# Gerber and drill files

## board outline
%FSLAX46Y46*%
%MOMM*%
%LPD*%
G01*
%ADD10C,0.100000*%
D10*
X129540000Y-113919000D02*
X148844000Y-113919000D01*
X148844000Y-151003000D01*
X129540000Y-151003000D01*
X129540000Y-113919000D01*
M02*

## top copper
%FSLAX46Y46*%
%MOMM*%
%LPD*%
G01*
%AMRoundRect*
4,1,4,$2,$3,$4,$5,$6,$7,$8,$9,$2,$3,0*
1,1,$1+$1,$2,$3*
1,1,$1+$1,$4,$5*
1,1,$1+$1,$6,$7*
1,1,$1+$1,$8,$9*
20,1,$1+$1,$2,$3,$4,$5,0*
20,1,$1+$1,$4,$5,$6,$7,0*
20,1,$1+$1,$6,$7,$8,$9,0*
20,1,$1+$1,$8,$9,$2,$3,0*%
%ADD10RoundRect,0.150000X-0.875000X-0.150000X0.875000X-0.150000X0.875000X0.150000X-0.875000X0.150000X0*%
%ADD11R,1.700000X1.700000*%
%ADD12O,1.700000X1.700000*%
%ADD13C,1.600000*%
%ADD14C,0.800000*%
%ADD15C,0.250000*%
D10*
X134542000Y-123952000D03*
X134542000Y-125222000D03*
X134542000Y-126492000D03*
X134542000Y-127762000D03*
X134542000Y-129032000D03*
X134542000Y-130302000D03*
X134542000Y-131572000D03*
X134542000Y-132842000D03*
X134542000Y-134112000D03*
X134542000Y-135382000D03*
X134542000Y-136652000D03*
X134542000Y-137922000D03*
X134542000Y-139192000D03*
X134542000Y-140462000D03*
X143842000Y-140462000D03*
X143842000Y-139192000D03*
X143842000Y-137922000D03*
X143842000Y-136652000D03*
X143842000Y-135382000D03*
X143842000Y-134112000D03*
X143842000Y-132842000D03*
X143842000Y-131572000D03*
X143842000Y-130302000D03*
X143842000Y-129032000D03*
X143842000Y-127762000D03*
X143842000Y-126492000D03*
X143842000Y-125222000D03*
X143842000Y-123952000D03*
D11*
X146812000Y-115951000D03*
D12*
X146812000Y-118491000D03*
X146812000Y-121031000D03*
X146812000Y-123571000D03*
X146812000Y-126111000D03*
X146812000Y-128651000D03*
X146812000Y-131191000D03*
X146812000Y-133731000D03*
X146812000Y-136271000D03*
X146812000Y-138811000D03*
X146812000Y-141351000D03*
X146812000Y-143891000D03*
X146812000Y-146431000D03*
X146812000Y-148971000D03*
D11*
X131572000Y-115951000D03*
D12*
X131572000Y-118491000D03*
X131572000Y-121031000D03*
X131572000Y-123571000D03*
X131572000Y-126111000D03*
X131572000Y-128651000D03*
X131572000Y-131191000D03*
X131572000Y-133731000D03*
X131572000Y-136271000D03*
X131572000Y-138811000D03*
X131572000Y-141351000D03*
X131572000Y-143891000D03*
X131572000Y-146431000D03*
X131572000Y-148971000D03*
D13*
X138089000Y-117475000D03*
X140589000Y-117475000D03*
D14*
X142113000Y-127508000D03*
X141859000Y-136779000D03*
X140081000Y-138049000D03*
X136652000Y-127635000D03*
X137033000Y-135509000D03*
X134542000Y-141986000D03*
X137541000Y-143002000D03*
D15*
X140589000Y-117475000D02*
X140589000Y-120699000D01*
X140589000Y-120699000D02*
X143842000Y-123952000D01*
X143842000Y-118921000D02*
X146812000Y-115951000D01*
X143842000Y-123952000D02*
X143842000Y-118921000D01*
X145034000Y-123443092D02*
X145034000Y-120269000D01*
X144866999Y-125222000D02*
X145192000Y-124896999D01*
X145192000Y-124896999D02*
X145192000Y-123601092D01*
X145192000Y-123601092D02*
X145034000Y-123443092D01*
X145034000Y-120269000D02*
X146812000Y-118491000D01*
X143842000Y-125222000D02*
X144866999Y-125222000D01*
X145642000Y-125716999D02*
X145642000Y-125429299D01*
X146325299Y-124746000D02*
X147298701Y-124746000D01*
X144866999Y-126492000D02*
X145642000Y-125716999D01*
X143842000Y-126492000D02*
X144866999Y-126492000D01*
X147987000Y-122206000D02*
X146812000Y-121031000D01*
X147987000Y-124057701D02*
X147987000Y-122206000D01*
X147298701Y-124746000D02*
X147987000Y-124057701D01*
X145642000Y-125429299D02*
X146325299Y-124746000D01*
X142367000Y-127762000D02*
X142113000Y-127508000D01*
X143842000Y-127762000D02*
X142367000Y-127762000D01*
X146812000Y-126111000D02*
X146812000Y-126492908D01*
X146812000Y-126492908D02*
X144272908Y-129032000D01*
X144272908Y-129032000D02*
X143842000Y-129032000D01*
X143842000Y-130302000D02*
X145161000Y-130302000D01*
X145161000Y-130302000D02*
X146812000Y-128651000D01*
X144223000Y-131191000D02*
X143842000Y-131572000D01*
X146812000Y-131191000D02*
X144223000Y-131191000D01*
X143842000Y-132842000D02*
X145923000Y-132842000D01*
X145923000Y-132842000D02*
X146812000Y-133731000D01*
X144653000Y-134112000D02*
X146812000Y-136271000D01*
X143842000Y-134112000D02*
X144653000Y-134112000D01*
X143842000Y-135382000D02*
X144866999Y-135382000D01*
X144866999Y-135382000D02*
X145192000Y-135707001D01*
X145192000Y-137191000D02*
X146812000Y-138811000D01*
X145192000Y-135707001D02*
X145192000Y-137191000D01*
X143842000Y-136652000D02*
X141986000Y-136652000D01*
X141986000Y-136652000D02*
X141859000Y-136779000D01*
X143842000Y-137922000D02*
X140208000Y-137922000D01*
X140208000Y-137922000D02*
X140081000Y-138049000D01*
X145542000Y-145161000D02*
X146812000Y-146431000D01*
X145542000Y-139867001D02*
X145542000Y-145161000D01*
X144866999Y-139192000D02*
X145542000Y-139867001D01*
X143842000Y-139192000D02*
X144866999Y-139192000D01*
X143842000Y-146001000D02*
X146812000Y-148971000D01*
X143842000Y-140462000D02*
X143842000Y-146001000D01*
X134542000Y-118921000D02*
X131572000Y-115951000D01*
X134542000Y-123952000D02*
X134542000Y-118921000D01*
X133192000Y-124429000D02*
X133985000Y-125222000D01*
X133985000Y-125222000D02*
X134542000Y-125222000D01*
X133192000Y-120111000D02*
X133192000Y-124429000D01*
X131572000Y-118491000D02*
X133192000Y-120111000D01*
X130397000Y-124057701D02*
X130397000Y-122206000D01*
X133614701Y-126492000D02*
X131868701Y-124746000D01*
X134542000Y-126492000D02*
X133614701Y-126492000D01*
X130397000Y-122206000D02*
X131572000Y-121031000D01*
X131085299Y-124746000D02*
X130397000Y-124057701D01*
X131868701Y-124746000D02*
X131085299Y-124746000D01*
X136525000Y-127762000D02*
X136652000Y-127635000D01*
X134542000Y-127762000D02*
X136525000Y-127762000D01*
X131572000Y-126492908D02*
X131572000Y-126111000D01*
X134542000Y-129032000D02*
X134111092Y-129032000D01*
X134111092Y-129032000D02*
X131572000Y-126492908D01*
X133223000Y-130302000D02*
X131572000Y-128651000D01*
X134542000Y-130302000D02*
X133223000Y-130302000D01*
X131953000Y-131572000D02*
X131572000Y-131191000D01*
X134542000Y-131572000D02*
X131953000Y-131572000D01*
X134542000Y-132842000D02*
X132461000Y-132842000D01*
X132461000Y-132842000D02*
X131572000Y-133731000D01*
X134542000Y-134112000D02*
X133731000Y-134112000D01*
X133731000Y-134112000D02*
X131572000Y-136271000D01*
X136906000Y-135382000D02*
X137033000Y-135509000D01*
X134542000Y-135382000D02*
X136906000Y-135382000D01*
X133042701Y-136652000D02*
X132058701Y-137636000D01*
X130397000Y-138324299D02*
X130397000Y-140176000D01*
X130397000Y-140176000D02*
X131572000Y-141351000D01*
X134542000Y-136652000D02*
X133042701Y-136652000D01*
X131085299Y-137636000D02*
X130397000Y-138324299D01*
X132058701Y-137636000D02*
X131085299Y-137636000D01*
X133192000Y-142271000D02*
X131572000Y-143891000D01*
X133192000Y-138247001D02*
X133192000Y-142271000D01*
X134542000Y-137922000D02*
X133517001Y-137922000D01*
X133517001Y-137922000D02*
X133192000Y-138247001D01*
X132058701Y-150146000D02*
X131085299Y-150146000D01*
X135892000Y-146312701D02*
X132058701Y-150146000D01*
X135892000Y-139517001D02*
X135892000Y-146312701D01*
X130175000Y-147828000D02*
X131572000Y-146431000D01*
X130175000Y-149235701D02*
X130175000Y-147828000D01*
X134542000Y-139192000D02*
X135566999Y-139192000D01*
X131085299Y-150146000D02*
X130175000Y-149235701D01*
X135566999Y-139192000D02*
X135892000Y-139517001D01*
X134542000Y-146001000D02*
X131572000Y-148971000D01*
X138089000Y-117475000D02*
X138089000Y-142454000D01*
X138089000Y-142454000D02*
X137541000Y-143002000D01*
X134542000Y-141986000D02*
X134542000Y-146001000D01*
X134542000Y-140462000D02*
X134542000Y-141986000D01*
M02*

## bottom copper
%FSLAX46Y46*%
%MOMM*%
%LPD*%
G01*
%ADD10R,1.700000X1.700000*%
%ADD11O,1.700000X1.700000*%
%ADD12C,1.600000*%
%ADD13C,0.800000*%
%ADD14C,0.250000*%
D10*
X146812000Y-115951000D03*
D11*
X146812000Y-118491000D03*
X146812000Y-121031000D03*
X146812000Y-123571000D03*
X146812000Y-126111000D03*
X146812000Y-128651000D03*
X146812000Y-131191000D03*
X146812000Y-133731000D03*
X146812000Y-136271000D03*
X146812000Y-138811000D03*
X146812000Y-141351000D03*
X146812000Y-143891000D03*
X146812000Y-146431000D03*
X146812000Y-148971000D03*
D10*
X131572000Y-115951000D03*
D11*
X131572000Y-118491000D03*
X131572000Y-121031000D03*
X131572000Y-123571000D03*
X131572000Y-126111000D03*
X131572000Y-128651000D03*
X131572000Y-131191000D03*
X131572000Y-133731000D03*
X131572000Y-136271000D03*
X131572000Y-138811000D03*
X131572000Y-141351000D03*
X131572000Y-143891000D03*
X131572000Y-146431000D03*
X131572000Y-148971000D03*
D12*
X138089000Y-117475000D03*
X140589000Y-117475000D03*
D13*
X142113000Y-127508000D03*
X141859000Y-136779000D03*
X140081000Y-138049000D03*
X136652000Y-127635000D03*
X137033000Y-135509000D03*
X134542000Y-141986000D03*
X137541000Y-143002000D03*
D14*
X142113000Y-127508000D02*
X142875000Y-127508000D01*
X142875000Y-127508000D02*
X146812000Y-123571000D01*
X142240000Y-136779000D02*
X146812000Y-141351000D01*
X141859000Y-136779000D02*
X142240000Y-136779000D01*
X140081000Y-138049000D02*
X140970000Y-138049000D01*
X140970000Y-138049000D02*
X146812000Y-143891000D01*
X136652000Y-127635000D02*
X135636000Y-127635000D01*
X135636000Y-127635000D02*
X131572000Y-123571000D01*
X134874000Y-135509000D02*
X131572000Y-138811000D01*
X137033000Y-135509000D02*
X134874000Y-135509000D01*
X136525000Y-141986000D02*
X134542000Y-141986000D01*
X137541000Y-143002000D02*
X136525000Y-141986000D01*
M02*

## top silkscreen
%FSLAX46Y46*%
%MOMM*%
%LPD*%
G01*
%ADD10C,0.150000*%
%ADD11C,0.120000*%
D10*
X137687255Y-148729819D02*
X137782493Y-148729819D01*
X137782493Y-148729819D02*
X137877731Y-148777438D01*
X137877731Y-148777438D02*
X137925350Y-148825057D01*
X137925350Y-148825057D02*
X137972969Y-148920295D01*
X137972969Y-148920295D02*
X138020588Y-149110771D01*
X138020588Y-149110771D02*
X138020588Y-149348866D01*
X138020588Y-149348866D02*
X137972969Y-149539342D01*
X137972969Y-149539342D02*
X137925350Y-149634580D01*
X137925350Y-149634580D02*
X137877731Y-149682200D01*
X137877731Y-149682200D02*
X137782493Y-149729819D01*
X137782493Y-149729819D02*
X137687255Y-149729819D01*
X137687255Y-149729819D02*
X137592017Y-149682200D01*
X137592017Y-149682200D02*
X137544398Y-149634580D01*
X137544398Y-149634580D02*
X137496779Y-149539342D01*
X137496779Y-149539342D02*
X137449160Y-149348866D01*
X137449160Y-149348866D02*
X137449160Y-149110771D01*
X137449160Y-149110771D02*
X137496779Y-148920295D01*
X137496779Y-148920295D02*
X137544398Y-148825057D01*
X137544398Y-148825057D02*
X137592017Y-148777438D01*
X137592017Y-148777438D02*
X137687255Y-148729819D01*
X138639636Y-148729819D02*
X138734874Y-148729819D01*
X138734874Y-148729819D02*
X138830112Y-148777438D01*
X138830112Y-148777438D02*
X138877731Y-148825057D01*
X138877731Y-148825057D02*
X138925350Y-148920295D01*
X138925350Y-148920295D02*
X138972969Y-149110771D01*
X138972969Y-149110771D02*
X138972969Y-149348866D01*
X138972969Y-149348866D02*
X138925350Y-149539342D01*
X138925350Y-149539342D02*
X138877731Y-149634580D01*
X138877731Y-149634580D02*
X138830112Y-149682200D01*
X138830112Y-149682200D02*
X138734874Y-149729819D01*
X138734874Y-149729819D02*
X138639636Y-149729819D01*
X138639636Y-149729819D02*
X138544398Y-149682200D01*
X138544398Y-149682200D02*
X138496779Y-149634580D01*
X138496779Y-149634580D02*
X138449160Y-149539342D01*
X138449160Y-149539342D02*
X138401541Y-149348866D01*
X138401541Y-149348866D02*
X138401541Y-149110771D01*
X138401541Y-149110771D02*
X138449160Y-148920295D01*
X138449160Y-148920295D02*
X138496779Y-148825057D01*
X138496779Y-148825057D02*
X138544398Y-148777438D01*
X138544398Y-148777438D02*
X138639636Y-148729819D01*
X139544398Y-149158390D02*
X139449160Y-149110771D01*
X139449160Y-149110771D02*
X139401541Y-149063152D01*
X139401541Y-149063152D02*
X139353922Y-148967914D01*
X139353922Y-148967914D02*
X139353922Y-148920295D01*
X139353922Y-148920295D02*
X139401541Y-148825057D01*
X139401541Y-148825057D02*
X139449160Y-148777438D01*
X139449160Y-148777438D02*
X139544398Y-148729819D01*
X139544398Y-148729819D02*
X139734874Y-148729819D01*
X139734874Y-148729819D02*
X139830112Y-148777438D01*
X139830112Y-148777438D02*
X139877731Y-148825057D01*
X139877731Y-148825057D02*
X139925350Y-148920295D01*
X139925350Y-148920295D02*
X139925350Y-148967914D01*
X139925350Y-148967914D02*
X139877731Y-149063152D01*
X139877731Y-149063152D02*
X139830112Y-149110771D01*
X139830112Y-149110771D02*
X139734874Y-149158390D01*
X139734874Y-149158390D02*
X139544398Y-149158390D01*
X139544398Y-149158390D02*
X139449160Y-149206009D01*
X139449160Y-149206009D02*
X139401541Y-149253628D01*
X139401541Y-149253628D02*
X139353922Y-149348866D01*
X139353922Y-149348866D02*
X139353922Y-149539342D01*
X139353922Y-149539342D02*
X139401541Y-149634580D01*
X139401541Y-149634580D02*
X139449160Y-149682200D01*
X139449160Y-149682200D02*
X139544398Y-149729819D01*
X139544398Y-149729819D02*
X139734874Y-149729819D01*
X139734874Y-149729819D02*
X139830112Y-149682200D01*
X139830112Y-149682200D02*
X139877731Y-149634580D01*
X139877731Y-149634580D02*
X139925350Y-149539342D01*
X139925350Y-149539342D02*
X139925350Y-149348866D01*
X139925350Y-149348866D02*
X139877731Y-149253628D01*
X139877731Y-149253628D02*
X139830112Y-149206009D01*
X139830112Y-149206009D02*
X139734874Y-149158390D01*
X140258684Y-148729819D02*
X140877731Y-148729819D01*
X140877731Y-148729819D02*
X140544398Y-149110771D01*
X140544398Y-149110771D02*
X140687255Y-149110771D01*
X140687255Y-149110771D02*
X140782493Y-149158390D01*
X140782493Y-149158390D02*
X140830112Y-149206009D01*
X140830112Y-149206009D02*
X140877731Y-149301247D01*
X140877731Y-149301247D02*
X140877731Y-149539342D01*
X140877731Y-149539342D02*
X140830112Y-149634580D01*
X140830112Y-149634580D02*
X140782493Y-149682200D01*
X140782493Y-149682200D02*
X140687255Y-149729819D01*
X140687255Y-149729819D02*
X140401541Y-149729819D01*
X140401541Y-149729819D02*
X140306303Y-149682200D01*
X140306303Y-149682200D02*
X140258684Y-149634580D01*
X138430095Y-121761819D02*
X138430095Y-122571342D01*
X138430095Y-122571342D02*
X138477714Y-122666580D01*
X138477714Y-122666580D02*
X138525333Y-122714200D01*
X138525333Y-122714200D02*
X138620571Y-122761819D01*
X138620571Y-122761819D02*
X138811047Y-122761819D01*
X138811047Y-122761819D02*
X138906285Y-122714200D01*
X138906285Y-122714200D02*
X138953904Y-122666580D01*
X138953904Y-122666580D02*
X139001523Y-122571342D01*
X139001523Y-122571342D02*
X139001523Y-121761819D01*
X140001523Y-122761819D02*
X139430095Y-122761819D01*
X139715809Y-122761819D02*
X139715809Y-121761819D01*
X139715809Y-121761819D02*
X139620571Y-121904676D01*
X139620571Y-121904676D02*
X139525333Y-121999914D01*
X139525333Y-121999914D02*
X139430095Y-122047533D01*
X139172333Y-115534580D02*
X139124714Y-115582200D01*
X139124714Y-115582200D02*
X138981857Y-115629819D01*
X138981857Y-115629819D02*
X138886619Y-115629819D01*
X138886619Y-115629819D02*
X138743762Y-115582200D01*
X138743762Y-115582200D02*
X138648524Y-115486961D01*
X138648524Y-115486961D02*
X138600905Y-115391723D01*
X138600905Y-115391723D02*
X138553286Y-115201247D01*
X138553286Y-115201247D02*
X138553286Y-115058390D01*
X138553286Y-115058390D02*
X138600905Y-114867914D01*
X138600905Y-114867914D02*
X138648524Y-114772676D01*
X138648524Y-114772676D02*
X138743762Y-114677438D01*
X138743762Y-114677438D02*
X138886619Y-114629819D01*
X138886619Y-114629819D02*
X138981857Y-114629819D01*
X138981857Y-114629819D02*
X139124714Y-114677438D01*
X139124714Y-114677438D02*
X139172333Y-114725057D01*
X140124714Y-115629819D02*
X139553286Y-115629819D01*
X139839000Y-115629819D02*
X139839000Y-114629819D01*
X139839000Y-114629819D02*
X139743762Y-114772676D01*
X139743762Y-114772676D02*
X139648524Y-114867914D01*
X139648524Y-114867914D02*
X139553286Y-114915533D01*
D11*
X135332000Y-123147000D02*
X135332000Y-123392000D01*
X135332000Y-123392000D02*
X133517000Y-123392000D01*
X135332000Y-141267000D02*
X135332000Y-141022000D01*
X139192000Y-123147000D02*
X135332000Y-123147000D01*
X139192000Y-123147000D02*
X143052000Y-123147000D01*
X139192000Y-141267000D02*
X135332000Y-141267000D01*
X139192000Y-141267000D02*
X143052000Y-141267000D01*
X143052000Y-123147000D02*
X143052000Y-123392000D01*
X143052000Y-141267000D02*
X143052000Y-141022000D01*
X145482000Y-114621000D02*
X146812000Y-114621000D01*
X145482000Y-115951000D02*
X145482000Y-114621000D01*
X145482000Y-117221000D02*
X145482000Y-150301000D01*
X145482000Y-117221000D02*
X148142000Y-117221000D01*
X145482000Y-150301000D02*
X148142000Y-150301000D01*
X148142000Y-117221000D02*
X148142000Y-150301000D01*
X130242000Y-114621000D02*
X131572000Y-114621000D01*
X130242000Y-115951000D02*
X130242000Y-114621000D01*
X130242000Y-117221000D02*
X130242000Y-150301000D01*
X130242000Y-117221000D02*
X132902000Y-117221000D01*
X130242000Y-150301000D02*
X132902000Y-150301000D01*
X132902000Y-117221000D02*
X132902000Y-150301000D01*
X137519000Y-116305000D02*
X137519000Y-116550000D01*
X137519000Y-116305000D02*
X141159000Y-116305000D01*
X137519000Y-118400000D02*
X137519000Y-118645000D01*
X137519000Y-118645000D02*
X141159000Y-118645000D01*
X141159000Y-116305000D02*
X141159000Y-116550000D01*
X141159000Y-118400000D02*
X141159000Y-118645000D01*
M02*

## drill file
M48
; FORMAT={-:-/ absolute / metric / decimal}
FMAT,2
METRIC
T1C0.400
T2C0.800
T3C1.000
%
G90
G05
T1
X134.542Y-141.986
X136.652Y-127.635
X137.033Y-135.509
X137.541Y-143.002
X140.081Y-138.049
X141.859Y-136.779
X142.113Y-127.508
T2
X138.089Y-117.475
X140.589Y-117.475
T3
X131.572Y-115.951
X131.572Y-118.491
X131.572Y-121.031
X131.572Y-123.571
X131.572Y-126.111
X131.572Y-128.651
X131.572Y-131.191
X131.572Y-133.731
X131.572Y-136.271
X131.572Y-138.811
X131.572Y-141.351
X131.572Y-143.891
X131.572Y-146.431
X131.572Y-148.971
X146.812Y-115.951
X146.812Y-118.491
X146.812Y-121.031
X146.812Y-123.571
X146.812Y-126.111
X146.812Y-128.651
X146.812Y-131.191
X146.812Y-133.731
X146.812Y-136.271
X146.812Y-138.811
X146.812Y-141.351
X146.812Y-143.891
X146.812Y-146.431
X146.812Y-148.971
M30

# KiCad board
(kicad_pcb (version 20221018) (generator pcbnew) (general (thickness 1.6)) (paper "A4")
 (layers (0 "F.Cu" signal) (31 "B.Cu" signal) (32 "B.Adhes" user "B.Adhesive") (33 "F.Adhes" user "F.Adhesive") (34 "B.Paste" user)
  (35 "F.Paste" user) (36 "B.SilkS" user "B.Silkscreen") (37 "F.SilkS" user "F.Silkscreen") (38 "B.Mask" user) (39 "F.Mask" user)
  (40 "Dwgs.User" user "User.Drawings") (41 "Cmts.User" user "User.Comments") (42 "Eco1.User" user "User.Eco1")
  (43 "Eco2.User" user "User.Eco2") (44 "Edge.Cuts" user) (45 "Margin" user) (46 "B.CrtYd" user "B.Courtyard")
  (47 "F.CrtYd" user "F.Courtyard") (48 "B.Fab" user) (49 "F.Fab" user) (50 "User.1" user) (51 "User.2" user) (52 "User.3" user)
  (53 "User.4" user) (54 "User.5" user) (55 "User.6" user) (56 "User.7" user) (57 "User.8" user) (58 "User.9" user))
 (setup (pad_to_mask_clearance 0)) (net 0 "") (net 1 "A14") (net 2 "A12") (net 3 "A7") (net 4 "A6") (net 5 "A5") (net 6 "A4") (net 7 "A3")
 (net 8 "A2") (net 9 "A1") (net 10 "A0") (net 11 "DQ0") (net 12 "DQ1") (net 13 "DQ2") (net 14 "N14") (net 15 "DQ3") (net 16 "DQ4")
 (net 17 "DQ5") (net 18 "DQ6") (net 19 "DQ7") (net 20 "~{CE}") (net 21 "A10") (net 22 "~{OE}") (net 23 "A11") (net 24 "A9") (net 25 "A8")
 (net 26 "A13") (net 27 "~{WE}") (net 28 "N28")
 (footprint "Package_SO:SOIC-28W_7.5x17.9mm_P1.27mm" (layer "F.Cu") (at 139.192 132.207)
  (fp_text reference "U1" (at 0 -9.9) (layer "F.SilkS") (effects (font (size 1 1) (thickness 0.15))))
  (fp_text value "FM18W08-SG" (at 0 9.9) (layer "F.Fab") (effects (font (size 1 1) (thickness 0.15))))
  (fp_line (start -3.86 -9.06) (end -3.86 -8.815) (stroke (width 0.12) (type solid)) (layer "F.SilkS"))
  (fp_line (start -3.86 -8.815) (end -5.675 -8.815) (stroke (width 0.12) (type solid)) (layer "F.SilkS"))
  (fp_line (start -3.86 9.06) (end -3.86 8.815) (stroke (width 0.12) (type solid)) (layer "F.SilkS"))
  (fp_line (start 0 -9.06) (end -3.86 -9.06) (stroke (width 0.12) (type solid)) (layer "F.SilkS"))
  (fp_line (start 0 -9.06) (end 3.86 -9.06) (stroke (width 0.12) (type solid)) (layer "F.SilkS"))
  (fp_line (start 0 9.06) (end -3.86 9.06) (stroke (width 0.12) (type solid)) (layer "F.SilkS"))
  (fp_line (start 0 9.06) (end 3.86 9.06) (stroke (width 0.12) (type solid)) (layer "F.SilkS"))
  (fp_line (start 3.86 -9.06) (end 3.86 -8.815) (stroke (width 0.12) (type solid)) (layer "F.SilkS"))
  (fp_line (start 3.86 9.06) (end 3.86 8.815) (stroke (width 0.12) (type solid)) (layer "F.SilkS"))
  (pad "1" smd roundrect (at -4.65 -8.255) (size 2.05 0.6) (layers "F.Cu" "F.Paste" "F.Mask") (roundrect_rratio 0.25) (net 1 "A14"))
  (pad "2" smd roundrect (at -4.65 -6.985) (size 2.05 0.6) (layers "F.Cu" "F.Paste" "F.Mask") (roundrect_rratio 0.25) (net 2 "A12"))
  (pad "3" smd roundrect (at -4.65 -5.715) (size 2.05 0.6) (layers "F.Cu" "F.Paste" "F.Mask") (roundrect_rratio 0.25) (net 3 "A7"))
  (pad "4" smd roundrect (at -4.65 -4.445) (size 2.05 0.6) (layers "F.Cu" "F.Paste" "F.Mask") (roundrect_rratio 0.25) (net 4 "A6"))
  (pad "5" smd roundrect (at -4.65 -3.175) (size 2.05 0.6) (layers "F.Cu" "F.Paste" "F.Mask") (roundrect_rratio 0.25) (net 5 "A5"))
  (pad "6" smd roundrect (at -4.65 -1.905) (size 2.05 0.6) (layers "F.Cu" "F.Paste" "F.Mask") (roundrect_rratio 0.25) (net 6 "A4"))
  (pad "7" smd roundrect (at -4.65 -0.635) (size 2.05 0.6) (layers "F.Cu" "F.Paste" "F.Mask") (roundrect_rratio 0.25) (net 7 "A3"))
  (pad "8" smd roundrect (at -4.65 0.635) (size 2.05 0.6) (layers "F.Cu" "F.Paste" "F.Mask") (roundrect_rratio 0.25) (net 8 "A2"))
  (pad "9" smd roundrect (at -4.65 1.905) (size 2.05 0.6) (layers "F.Cu" "F.Paste" "F.Mask") (roundrect_rratio 0.25) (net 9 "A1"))
  (pad "10" smd roundrect (at -4.65 3.175) (size 2.05 0.6) (layers "F.Cu" "F.Paste" "F.Mask") (roundrect_rratio 0.25) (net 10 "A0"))
  (pad "11" smd roundrect (at -4.65 4.445) (size 2.05 0.6) (layers "F.Cu" "F.Paste" "F.Mask") (roundrect_rratio 0.25) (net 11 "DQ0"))
  (pad "12" smd roundrect (at -4.65 5.715) (size 2.05 0.6) (layers "F.Cu" "F.Paste" "F.Mask") (roundrect_rratio 0.25) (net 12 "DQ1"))
  (pad "13" smd roundrect (at -4.65 6.985) (size 2.05 0.6) (layers "F.Cu" "F.Paste" "F.Mask") (roundrect_rratio 0.25) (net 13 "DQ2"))
  (pad "14" smd roundrect (at -4.65 8.255) (size 2.05 0.6) (layers "F.Cu" "F.Paste" "F.Mask") (roundrect_rratio 0.25) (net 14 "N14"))
  (pad "15" smd roundrect (at 4.65 8.255) (size 2.05 0.6) (layers "F.Cu" "F.Paste" "F.Mask") (roundrect_rratio 0.25) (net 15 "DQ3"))
  (pad "16" smd roundrect (at 4.65 6.985) (size 2.05 0.6) (layers "F.Cu" "F.Paste" "F.Mask") (roundrect_rratio 0.25) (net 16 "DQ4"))
  (pad "17" smd roundrect (at 4.65 5.715) (size 2.05 0.6) (layers "F.Cu" "F.Paste" "F.Mask") (roundrect_rratio 0.25) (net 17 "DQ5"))
  (pad "18" smd roundrect (at 4.65 4.445) (size 2.05 0.6) (layers "F.Cu" "F.Paste" "F.Mask") (roundrect_rratio 0.25) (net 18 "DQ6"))
  (pad "19" smd roundrect (at 4.65 3.175) (size 2.05 0.6) (layers "F.Cu" "F.Paste" "F.Mask") (roundrect_rratio 0.25) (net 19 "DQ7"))
  (pad "20" smd roundrect (at 4.65 1.905) (size 2.05 0.6) (layers "F.Cu" "F.Paste" "F.Mask") (roundrect_rratio 0.25) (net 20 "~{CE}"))
  (pad "21" smd roundrect (at 4.65 0.635) (size 2.05 0.6) (layers "F.Cu" "F.Paste" "F.Mask") (roundrect_rratio 0.25) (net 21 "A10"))
  (pad "22" smd roundrect (at 4.65 -0.635) (size 2.05 0.6) (layers "F.Cu" "F.Paste" "F.Mask") (roundrect_rratio 0.25) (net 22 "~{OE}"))
  (pad "23" smd roundrect (at 4.65 -1.905) (size 2.05 0.6) (layers "F.Cu" "F.Paste" "F.Mask") (roundrect_rratio 0.25) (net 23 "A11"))
  (pad "24" smd roundrect (at 4.65 -3.175) (size 2.05 0.6) (layers "F.Cu" "F.Paste" "F.Mask") (roundrect_rratio 0.25) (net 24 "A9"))
  (pad "25" smd roundrect (at 4.65 -4.445) (size 2.05 0.6) (layers "F.Cu" "F.Paste" "F.Mask") (roundrect_rratio 0.25) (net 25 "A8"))
  (pad "26" smd roundrect (at 4.65 -5.715) (size 2.05 0.6) (layers "F.Cu" "F.Paste" "F.Mask") (roundrect_rratio 0.25) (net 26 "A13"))
  (pad "27" smd roundrect (at 4.65 -6.985) (size 2.05 0.6) (layers "F.Cu" "F.Paste" "F.Mask") (roundrect_rratio 0.25) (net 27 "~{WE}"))
  (pad "28" smd roundrect (at 4.65 -8.255) (size 2.05 0.6) (layers "F.Cu" "F.Paste" "F.Mask") (roundrect_rratio 0.25) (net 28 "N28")))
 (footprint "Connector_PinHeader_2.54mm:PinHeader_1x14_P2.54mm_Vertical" (layer "F.Cu") (at 146.812 115.951)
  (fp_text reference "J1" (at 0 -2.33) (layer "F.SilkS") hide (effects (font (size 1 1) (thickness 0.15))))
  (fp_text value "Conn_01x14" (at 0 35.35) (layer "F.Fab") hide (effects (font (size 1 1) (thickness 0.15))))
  (fp_line (start -1.33 -1.33) (end 0 -1.33) (stroke (width 0.12) (type solid)) (layer "F.SilkS"))
  (fp_line (start -1.33 0) (end -1.33 -1.33) (stroke (width 0.12) (type solid)) (layer "F.SilkS"))
  (fp_line (start -1.33 1.27) (end -1.33 34.35) (stroke (width 0.12) (type solid)) (layer "F.SilkS"))
  (fp_line (start -1.33 1.27) (end 1.33 1.27) (stroke (width 0.12) (type solid)) (layer "F.SilkS"))
  (fp_line (start -1.33 34.35) (end 1.33 34.35) (stroke (width 0.12) (type solid)) (layer "F.SilkS"))
  (fp_line (start 1.33 1.27) (end 1.33 34.35) (stroke (width 0.12) (type solid)) (layer "F.SilkS"))
  (pad "1" thru_hole rect (at 0 0) (size 1.7 1.7) (drill 1) (layers "*.Cu" "*.Mask") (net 28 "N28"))
  (pad "2" thru_hole oval (at 0 2.54) (size 1.7 1.7) (drill 1) (layers "*.Cu" "*.Mask") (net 27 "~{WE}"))
  (pad "3" thru_hole oval (at 0 5.08) (size 1.7 1.7) (drill 1) (layers "*.Cu" "*.Mask") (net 26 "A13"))
  (pad "4" thru_hole oval (at 0 7.62) (size 1.7 1.7) (drill 1) (layers "*.Cu" "*.Mask") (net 25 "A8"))
  (pad "5" thru_hole oval (at 0 10.16) (size 1.7 1.7) (drill 1) (layers "*.Cu" "*.Mask") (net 24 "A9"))
  (pad "6" thru_hole oval (at 0 12.7) (size 1.7 1.7) (drill 1) (layers "*.Cu" "*.Mask") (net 23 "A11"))
  (pad "7" thru_hole oval (at 0 15.24) (size 1.7 1.7) (drill 1) (layers "*.Cu" "*.Mask") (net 22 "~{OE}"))
  (pad "8" thru_hole oval (at 0 17.78) (size 1.7 1.7) (drill 1) (layers "*.Cu" "*.Mask") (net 21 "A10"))
  (pad "9" thru_hole oval (at 0 20.32) (size 1.7 1.7) (drill 1) (layers "*.Cu" "*.Mask") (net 20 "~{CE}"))
  (pad "10" thru_hole oval (at 0 22.86) (size 1.7 1.7) (drill 1) (layers "*.Cu" "*.Mask") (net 19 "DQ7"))
  (pad "11" thru_hole oval (at 0 25.4) (size 1.7 1.7) (drill 1) (layers "*.Cu" "*.Mask") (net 18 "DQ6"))
  (pad "12" thru_hole oval (at 0 27.94) (size 1.7 1.7) (drill 1) (layers "*.Cu" "*.Mask") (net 17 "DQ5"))
  (pad "13" thru_hole oval (at 0 30.48) (size 1.7 1.7) (drill 1) (layers "*.Cu" "*.Mask") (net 16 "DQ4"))
  (pad "14" thru_hole oval (at 0 33.02) (size 1.7 1.7) (drill 1) (layers "*.Cu" "*.Mask") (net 15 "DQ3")))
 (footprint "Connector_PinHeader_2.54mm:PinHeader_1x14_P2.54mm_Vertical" (layer "F.Cu") (at 131.572 115.951)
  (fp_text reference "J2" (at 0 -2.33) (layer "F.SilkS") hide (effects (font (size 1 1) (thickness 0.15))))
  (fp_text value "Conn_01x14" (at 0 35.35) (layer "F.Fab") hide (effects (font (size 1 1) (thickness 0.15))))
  (fp_line (start -1.33 -1.33) (end 0 -1.33) (stroke (width 0.12) (type solid)) (layer "F.SilkS"))
  (fp_line (start -1.33 0) (end -1.33 -1.33) (stroke (width 0.12) (type solid)) (layer "F.SilkS"))
  (fp_line (start -1.33 1.27) (end -1.33 34.35) (stroke (width 0.12) (type solid)) (layer "F.SilkS"))
  (fp_line (start -1.33 1.27) (end 1.33 1.27) (stroke (width 0.12) (type solid)) (layer "F.SilkS"))
  (fp_line (start -1.33 34.35) (end 1.33 34.35) (stroke (width 0.12) (type solid)) (layer "F.SilkS"))
  (fp_line (start 1.33 1.27) (end 1.33 34.35) (stroke (width 0.12) (type solid)) (layer "F.SilkS"))
  (pad "1" thru_hole rect (at 0 0) (size 1.7 1.7) (drill 1) (layers "*.Cu" "*.Mask") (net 1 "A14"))
  (pad "2" thru_hole oval (at 0 2.54) (size 1.7 1.7) (drill 1) (layers "*.Cu" "*.Mask") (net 2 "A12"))
  (pad "3" thru_hole oval (at 0 5.08) (size 1.7 1.7) (drill 1) (layers "*.Cu" "*.Mask") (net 3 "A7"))
  (pad "4" thru_hole oval (at 0 7.62) (size 1.7 1.7) (drill 1) (layers "*.Cu" "*.Mask") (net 4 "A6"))
  (pad "5" thru_hole oval (at 0 10.16) (size 1.7 1.7) (drill 1) (layers "*.Cu" "*.Mask") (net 5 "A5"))
  (pad "6" thru_hole oval (at 0 12.7) (size 1.7 1.7) (drill 1) (layers "*.Cu" "*.Mask") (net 6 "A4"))
  (pad "7" thru_hole oval (at 0 15.24) (size 1.7 1.7) (drill 1) (layers "*.Cu" "*.Mask") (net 7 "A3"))
  (pad "8" thru_hole oval (at 0 17.78) (size 1.7 1.7) (drill 1) (layers "*.Cu" "*.Mask") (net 8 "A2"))
  (pad "9" thru_hole oval (at 0 20.32) (size 1.7 1.7) (drill 1) (layers "*.Cu" "*.Mask") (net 9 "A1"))
  (pad "10" thru_hole oval (at 0 22.86) (size 1.7 1.7) (drill 1) (layers "*.Cu" "*.Mask") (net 10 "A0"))
  (pad "11" thru_hole oval (at 0 25.4) (size 1.7 1.7) (drill 1) (layers "*.Cu" "*.Mask") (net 11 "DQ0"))
  (pad "12" thru_hole oval (at 0 27.94) (size 1.7 1.7) (drill 1) (layers "*.Cu" "*.Mask") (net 12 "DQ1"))
  (pad "13" thru_hole oval (at 0 30.48) (size 1.7 1.7) (drill 1) (layers "*.Cu" "*.Mask") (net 13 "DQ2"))
  (pad "14" thru_hole oval (at 0 33.02) (size 1.7 1.7) (drill 1) (layers "*.Cu" "*.Mask") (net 14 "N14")))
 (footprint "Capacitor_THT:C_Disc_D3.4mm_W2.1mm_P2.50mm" (layer "F.Cu") (at 138.089 117.475)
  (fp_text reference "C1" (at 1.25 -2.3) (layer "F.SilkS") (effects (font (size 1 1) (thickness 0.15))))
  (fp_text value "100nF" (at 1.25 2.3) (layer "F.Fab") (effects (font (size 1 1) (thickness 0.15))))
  (fp_line (start -0.57 -1.17) (end -0.57 -0.925) (stroke (width 0.12) (type solid)) (layer "F.SilkS"))
  (fp_line (start -0.57 -1.17) (end 3.07 -1.17) (stroke (width 0.12) (type solid)) (layer "F.SilkS"))
  (fp_line (start -0.57 0.925) (end -0.57 1.17) (stroke (width 0.12) (type solid)) (layer "F.SilkS"))
  (fp_line (start -0.57 1.17) (end 3.07 1.17) (stroke (width 0.12) (type solid)) (layer "F.SilkS"))
  (fp_line (start 3.07 -1.17) (end 3.07 -0.925) (stroke (width 0.12) (type solid)) (layer "F.SilkS"))
  (fp_line (start 3.07 0.925) (end 3.07 1.17) (stroke (width 0.12) (type solid)) (layer "F.SilkS"))
  (pad "1" thru_hole circle (at 0 0) (size 1.6 1.6) (drill 0.8) (layers "*.Cu" "*.Mask") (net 14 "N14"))
  (pad "2" thru_hole circle (at 2.5 0) (size 1.6 1.6) (drill 0.8) (layers "*.Cu" "*.Mask") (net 28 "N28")))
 (gr_rect (start 129.54 113.919) (end 148.844 151.003) (stroke (width 0.1) (type default)) (fill none) (layer "Edge.Cuts"))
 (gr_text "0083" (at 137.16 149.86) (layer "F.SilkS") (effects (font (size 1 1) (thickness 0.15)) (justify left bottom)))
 (segment (start 140.589 117.475) (end 140.589 120.699) (width 0.25) (layer "F.Cu") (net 28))
 (segment (start 140.589 120.699) (end 143.842 123.952) (width 0.25) (layer "F.Cu") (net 28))
 (segment (start 143.842 118.921) (end 146.812 115.951) (width 0.25) (layer "F.Cu") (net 28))
 (segment (start 143.842 123.952) (end 143.842 118.921) (width 0.25) (layer "F.Cu") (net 28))
 (segment (start 145.034 123.443092) (end 145.034 120.269) (width 0.25) (layer "F.Cu") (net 27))
 (segment (start 144.866999 125.222) (end 145.192 124.896999) (width 0.25) (layer "F.Cu") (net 27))
 (segment (start 145.192 124.896999) (end 145.192 123.601092) (width 0.25) (layer "F.Cu") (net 27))
 (segment (start 145.192 123.601092) (end 145.034 123.443092) (width 0.25) (layer "F.Cu") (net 27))
 (segment (start 145.034 120.269) (end 146.812 118.491) (width 0.25) (layer "F.Cu") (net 27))
 (segment (start 143.842 125.222) (end 144.866999 125.222) (width 0.25) (layer "F.Cu") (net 27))
 (segment (start 145.642 125.716999) (end 145.642 125.429299) (width 0.25) (layer "F.Cu") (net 26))
 (segment (start 146.325299 124.746) (end 147.298701 124.746) (width 0.25) (layer "F.Cu") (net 26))
 (segment (start 144.866999 126.492) (end 145.642 125.716999) (width 0.25) (layer "F.Cu") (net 26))
 (segment (start 143.842 126.492) (end 144.866999 126.492) (width 0.25) (layer "F.Cu") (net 26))
 (segment (start 147.987 122.206) (end 146.812 121.031) (width 0.25) (layer "F.Cu") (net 26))
 (segment (start 147.987 124.057701) (end 147.987 122.206) (width 0.25) (layer "F.Cu") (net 26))
 (segment (start 147.298701 124.746) (end 147.987 124.057701) (width 0.25) (layer "F.Cu") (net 26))
 (segment (start 145.642 125.429299) (end 146.325299 124.746) (width 0.25) (layer "F.Cu") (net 26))
 (segment (start 142.367 127.762) (end 142.113 127.508) (width 0.25) (layer "F.Cu") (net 25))
 (segment (start 143.842 127.762) (end 142.367 127.762) (width 0.25) (layer "F.Cu") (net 25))
 (via (at 142.113 127.508) (size 0.8) (drill 0.4) (layers "F.Cu" "B.Cu") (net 25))
 (segment (start 142.113 127.508) (end 142.875 127.508) (width 0.25) (layer "B.Cu") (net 25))
 (segment (start 142.875 127.508) (end 146.812 123.571) (width 0.25) (layer "B.Cu") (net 25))
 (segment (start 146.812 126.111) (end 146.812 126.492908) (width 0.25) (layer "F.Cu") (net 24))
 (segment (start 146.812 126.492908) (end 144.272908 129.032) (width 0.25) (layer "F.Cu") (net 24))
 (segment (start 144.272908 129.032) (end 143.842 129.032) (width 0.25) (layer "F.Cu") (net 24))
 (segment (start 143.842 130.302) (end 145.161 130.302) (width 0.25) (layer "F.Cu") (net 23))
 (segment (start 145.161 130.302) (end 146.812 128.651) (width 0.25) (layer "F.Cu") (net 23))
 (segment (start 144.223 131.191) (end 143.842 131.572) (width 0.25) (layer "F.Cu") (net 22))
 (segment (start 146.812 131.191) (end 144.223 131.191) (width 0.25) (layer "F.Cu") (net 22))
 (segment (start 143.842 132.842) (end 145.923 132.842) (width 0.25) (layer "F.Cu") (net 21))
 (segment (start 145.923 132.842) (end 146.812 133.731) (width 0.25) (layer "F.Cu") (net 21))
 (segment (start 144.653 134.112) (end 146.812 136.271) (width 0.25) (layer "F.Cu") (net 20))
 (segment (start 143.842 134.112) (end 144.653 134.112) (width 0.25) (layer "F.Cu") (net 20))
 (segment (start 143.842 135.382) (end 144.866999 135.382) (width 0.25) (layer "F.Cu") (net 19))
 (segment (start 144.866999 135.382) (end 145.192 135.707001) (width 0.25) (layer "F.Cu") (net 19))
 (segment (start 145.192 137.191) (end 146.812 138.811) (width 0.25) (layer "F.Cu") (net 19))
 (segment (start 145.192 135.707001) (end 145.192 137.191) (width 0.25) (layer "F.Cu") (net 19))
 (segment (start 143.842 136.652) (end 141.986 136.652) (width 0.25) (layer "F.Cu") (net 18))
 (segment (start 141.986 136.652) (end 141.859 136.779) (width 0.25) (layer "F.Cu") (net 18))
 (via (at 141.859 136.779) (size 0.8) (drill 0.4) (layers "F.Cu" "B.Cu") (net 18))
 (segment (start 142.24 136.779) (end 146.812 141.351) (width 0.25) (layer "B.Cu") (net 18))
 (segment (start 141.859 136.779) (end 142.24 136.779) (width 0.25) (layer "B.Cu") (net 18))
 (segment (start 143.842 137.922) (end 140.208 137.922) (width 0.25) (layer "F.Cu") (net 17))
 (segment (start 140.208 137.922) (end 140.081 138.049) (width 0.25) (layer "F.Cu") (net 17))
 (via (at 140.081 138.049) (size 0.8) (drill 0.4) (layers "F.Cu" "B.Cu") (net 17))
 (segment (start 140.081 138.049) (end 140.97 138.049) (width 0.25) (layer "B.Cu") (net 17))
 (segment (start 140.97 138.049) (end 146.812 143.891) (width 0.25) (layer "B.Cu") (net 17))
 (segment (start 145.542 145.161) (end 146.812 146.431) (width 0.25) (layer "F.Cu") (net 16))
 (segment (start 145.542 139.867001) (end 145.542 145.161) (width 0.25) (layer "F.Cu") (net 16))
 (segment (start 144.866999 139.192) (end 145.542 139.867001) (width 0.25) (layer "F.Cu") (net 16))
 (segment (start 143.842 139.192) (end 144.866999 139.192) (width 0.25) (layer "F.Cu") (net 16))
 (segment (start 143.842 146.001) (end 146.812 148.971) (width 0.25) (layer "F.Cu") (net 15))
 (segment (start 143.842 140.462) (end 143.842 146.001) (width 0.25) (layer "F.Cu") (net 15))
 (segment (start 134.542 118.921) (end 131.572 115.951) (width 0.25) (layer "F.Cu") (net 1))
 (segment (start 134.542 123.952) (end 134.542 118.921) (width 0.25) (layer "F.Cu") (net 1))
 (segment (start 133.192 124.429) (end 133.985 125.222) (width 0.25) (layer "F.Cu") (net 2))
 (segment (start 133.985 125.222) (end 134.542 125.222) (width 0.25) (layer "F.Cu") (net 2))
 (segment (start 133.192 120.111) (end 133.192 124.429) (width 0.25) (layer "F.Cu") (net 2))
 (segment (start 131.572 118.491) (end 133.192 120.111) (width 0.25) (layer "F.Cu") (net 2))
 (segment (start 130.397 124.057701) (end 130.397 122.206) (width 0.25) (layer "F.Cu") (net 3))
 (segment (start 133.614701 126.492) (end 131.868701 124.746) (width 0.25) (layer "F.Cu") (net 3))
 (segment (start 134.542 126.492) (end 133.614701 126.492) (width 0.25) (layer "F.Cu") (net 3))
 (segment (start 130.397 122.206) (end 131.572 121.031) (width 0.25) (layer "F.Cu") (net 3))
 (segment (start 131.085299 124.746) (end 130.397 124.057701) (width 0.25) (layer "F.Cu") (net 3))
 (segment (start 131.868701 124.746) (end 131.085299 124.746) (width 0.25) (layer "F.Cu") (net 3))
 (segment (start 136.525 127.762) (end 136.652 127.635) (width 0.25) (layer "F.Cu") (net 4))
 (segment (start 134.542 127.762) (end 136.525 127.762) (width 0.25) (layer "F.Cu") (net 4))
 (via (at 136.652 127.635) (size 0.8) (drill 0.4) (layers "F.Cu" "B.Cu") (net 4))
 (segment (start 136.652 127.635) (end 135.636 127.635) (width 0.25) (layer "B.Cu") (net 4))
 (segment (start 135.636 127.635) (end 131.572 123.571) (width 0.25) (layer "B.Cu") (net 4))
 (segment (start 131.572 126.492908) (end 131.572 126.111) (width 0.25) (layer "F.Cu") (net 5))
 (segment (start 134.542 129.032) (end 134.111092 129.032) (width 0.25) (layer "F.Cu") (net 5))
 (segment (start 134.111092 129.032) (end 131.572 126.492908) (width 0.25) (layer "F.Cu") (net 5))
 (segment (start 133.223 130.302) (end 131.572 128.651) (width 0.25) (layer "F.Cu") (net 6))
 (segment (start 134.542 130.302) (end 133.223 130.302) (width 0.25) (layer "F.Cu") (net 6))
 (segment (start 131.953 131.572) (end 131.572 131.191) (width 0.25) (layer "F.Cu") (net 7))
 (segment (start 134.542 131.572) (end 131.953 131.572) (width 0.25) (layer "F.Cu") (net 7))
 (segment (start 134.542 132.842) (end 132.461 132.842) (width 0.25) (layer "F.Cu") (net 8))
 (segment (start 132.461 132.842) (end 131.572 133.731) (width 0.25) (layer "F.Cu") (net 8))
 (segment (start 134.542 134.112) (end 133.731 134.112) (width 0.25) (layer "F.Cu") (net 9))
 (segment (start 133.731 134.112) (end 131.572 136.271) (width 0.25) (layer "F.Cu") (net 9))
 (segment (start 136.906 135.382) (end 137.033 135.509) (width 0.25) (layer "F.Cu") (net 10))
 (segment (start 134.542 135.382) (end 136.906 135.382) (width 0.25) (layer "F.Cu") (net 10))
 (via (at 137.033 135.509) (size 0.8) (drill 0.4) (layers "F.Cu" "B.Cu") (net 10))
 (segment (start 134.874 135.509) (end 131.572 138.811) (width 0.25) (layer "B.Cu") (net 10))
 (segment (start 137.033 135.509) (end 134.874 135.509) (width 0.25) (layer "B.Cu") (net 10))
 (segment (start 133.042701 136.652) (end 132.058701 137.636) (width 0.25) (layer "F.Cu") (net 11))
 (segment (start 130.397 138.324299) (end 130.397 140.176) (width 0.25) (layer "F.Cu") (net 11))
 (segment (start 130.397 140.176) (end 131.572 141.351) (width 0.25) (layer "F.Cu") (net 11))
 (segment (start 134.542 136.652) (end 133.042701 136.652) (width 0.25) (layer "F.Cu") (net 11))
 (segment (start 131.085299 137.636) (end 130.397 138.324299) (width 0.25) (layer "F.Cu") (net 11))
 (segment (start 132.058701 137.636) (end 131.085299 137.636) (width 0.25) (layer "F.Cu") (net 11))
 (segment (start 133.192 142.271) (end 131.572 143.891) (width 0.25) (layer "F.Cu") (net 12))
 (segment (start 133.192 138.247001) (end 133.192 142.271) (width 0.25) (layer "F.Cu") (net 12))
 (segment (start 134.542 137.922) (end 133.517001 137.922) (width 0.25) (layer "F.Cu") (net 12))
 (segment (start 133.517001 137.922) (end 133.192 138.247001) (width 0.25) (layer "F.Cu") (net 12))
 (segment (start 132.058701 150.146) (end 131.085299 150.146) (width 0.25) (layer "F.Cu") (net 13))
 (segment (start 135.892 146.312701) (end 132.058701 150.146) (width 0.25) (layer "F.Cu") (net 13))
 (segment (start 135.892 139.517001) (end 135.892 146.312701) (width 0.25) (layer "F.Cu") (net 13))
 (segment (start 130.175 147.828) (end 131.572 146.431) (width 0.25) (layer "F.Cu") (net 13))
 (segment (start 130.175 149.235701) (end 130.175 147.828) (width 0.25) (layer "F.Cu") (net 13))
 (segment (start 134.542 139.192) (end 135.566999 139.192) (width 0.25) (layer "F.Cu") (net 13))
 (segment (start 131.085299 150.146) (end 130.175 149.235701) (width 0.25) (layer "F.Cu") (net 13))
 (segment (start 135.566999 139.192) (end 135.892 139.517001) (width 0.25) (layer "F.Cu") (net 13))
 (segment (start 134.542 146.001) (end 131.572 148.971) (width 0.25) (layer "F.Cu") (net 14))
 (segment (start 138.089 117.475) (end 138.089 142.454) (width 0.25) (layer "F.Cu") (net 14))
 (segment (start 138.089 142.454) (end 137.541 143.002) (width 0.25) (layer "F.Cu") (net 14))
 (segment (start 134.542 141.986) (end 134.542 146.001) (width 0.25) (layer "F.Cu") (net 14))
 (segment (start 134.542 140.462) (end 134.542 141.986) (width 0.25) (layer "F.Cu") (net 14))
 (via (at 134.542 141.986) (size 0.8) (drill 0.4) (layers "F.Cu" "B.Cu") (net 14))
 (via (at 137.541 143.002) (size 0.8) (drill 0.4) (layers "F.Cu" "B.Cu") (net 14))
 (segment (start 136.525 141.986) (end 134.542 141.986) (width 0.25) (layer "B.Cu") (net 14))
 (segment (start 137.541 143.002) (end 136.525 141.986) (width 0.25) (layer "B.Cu") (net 14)))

